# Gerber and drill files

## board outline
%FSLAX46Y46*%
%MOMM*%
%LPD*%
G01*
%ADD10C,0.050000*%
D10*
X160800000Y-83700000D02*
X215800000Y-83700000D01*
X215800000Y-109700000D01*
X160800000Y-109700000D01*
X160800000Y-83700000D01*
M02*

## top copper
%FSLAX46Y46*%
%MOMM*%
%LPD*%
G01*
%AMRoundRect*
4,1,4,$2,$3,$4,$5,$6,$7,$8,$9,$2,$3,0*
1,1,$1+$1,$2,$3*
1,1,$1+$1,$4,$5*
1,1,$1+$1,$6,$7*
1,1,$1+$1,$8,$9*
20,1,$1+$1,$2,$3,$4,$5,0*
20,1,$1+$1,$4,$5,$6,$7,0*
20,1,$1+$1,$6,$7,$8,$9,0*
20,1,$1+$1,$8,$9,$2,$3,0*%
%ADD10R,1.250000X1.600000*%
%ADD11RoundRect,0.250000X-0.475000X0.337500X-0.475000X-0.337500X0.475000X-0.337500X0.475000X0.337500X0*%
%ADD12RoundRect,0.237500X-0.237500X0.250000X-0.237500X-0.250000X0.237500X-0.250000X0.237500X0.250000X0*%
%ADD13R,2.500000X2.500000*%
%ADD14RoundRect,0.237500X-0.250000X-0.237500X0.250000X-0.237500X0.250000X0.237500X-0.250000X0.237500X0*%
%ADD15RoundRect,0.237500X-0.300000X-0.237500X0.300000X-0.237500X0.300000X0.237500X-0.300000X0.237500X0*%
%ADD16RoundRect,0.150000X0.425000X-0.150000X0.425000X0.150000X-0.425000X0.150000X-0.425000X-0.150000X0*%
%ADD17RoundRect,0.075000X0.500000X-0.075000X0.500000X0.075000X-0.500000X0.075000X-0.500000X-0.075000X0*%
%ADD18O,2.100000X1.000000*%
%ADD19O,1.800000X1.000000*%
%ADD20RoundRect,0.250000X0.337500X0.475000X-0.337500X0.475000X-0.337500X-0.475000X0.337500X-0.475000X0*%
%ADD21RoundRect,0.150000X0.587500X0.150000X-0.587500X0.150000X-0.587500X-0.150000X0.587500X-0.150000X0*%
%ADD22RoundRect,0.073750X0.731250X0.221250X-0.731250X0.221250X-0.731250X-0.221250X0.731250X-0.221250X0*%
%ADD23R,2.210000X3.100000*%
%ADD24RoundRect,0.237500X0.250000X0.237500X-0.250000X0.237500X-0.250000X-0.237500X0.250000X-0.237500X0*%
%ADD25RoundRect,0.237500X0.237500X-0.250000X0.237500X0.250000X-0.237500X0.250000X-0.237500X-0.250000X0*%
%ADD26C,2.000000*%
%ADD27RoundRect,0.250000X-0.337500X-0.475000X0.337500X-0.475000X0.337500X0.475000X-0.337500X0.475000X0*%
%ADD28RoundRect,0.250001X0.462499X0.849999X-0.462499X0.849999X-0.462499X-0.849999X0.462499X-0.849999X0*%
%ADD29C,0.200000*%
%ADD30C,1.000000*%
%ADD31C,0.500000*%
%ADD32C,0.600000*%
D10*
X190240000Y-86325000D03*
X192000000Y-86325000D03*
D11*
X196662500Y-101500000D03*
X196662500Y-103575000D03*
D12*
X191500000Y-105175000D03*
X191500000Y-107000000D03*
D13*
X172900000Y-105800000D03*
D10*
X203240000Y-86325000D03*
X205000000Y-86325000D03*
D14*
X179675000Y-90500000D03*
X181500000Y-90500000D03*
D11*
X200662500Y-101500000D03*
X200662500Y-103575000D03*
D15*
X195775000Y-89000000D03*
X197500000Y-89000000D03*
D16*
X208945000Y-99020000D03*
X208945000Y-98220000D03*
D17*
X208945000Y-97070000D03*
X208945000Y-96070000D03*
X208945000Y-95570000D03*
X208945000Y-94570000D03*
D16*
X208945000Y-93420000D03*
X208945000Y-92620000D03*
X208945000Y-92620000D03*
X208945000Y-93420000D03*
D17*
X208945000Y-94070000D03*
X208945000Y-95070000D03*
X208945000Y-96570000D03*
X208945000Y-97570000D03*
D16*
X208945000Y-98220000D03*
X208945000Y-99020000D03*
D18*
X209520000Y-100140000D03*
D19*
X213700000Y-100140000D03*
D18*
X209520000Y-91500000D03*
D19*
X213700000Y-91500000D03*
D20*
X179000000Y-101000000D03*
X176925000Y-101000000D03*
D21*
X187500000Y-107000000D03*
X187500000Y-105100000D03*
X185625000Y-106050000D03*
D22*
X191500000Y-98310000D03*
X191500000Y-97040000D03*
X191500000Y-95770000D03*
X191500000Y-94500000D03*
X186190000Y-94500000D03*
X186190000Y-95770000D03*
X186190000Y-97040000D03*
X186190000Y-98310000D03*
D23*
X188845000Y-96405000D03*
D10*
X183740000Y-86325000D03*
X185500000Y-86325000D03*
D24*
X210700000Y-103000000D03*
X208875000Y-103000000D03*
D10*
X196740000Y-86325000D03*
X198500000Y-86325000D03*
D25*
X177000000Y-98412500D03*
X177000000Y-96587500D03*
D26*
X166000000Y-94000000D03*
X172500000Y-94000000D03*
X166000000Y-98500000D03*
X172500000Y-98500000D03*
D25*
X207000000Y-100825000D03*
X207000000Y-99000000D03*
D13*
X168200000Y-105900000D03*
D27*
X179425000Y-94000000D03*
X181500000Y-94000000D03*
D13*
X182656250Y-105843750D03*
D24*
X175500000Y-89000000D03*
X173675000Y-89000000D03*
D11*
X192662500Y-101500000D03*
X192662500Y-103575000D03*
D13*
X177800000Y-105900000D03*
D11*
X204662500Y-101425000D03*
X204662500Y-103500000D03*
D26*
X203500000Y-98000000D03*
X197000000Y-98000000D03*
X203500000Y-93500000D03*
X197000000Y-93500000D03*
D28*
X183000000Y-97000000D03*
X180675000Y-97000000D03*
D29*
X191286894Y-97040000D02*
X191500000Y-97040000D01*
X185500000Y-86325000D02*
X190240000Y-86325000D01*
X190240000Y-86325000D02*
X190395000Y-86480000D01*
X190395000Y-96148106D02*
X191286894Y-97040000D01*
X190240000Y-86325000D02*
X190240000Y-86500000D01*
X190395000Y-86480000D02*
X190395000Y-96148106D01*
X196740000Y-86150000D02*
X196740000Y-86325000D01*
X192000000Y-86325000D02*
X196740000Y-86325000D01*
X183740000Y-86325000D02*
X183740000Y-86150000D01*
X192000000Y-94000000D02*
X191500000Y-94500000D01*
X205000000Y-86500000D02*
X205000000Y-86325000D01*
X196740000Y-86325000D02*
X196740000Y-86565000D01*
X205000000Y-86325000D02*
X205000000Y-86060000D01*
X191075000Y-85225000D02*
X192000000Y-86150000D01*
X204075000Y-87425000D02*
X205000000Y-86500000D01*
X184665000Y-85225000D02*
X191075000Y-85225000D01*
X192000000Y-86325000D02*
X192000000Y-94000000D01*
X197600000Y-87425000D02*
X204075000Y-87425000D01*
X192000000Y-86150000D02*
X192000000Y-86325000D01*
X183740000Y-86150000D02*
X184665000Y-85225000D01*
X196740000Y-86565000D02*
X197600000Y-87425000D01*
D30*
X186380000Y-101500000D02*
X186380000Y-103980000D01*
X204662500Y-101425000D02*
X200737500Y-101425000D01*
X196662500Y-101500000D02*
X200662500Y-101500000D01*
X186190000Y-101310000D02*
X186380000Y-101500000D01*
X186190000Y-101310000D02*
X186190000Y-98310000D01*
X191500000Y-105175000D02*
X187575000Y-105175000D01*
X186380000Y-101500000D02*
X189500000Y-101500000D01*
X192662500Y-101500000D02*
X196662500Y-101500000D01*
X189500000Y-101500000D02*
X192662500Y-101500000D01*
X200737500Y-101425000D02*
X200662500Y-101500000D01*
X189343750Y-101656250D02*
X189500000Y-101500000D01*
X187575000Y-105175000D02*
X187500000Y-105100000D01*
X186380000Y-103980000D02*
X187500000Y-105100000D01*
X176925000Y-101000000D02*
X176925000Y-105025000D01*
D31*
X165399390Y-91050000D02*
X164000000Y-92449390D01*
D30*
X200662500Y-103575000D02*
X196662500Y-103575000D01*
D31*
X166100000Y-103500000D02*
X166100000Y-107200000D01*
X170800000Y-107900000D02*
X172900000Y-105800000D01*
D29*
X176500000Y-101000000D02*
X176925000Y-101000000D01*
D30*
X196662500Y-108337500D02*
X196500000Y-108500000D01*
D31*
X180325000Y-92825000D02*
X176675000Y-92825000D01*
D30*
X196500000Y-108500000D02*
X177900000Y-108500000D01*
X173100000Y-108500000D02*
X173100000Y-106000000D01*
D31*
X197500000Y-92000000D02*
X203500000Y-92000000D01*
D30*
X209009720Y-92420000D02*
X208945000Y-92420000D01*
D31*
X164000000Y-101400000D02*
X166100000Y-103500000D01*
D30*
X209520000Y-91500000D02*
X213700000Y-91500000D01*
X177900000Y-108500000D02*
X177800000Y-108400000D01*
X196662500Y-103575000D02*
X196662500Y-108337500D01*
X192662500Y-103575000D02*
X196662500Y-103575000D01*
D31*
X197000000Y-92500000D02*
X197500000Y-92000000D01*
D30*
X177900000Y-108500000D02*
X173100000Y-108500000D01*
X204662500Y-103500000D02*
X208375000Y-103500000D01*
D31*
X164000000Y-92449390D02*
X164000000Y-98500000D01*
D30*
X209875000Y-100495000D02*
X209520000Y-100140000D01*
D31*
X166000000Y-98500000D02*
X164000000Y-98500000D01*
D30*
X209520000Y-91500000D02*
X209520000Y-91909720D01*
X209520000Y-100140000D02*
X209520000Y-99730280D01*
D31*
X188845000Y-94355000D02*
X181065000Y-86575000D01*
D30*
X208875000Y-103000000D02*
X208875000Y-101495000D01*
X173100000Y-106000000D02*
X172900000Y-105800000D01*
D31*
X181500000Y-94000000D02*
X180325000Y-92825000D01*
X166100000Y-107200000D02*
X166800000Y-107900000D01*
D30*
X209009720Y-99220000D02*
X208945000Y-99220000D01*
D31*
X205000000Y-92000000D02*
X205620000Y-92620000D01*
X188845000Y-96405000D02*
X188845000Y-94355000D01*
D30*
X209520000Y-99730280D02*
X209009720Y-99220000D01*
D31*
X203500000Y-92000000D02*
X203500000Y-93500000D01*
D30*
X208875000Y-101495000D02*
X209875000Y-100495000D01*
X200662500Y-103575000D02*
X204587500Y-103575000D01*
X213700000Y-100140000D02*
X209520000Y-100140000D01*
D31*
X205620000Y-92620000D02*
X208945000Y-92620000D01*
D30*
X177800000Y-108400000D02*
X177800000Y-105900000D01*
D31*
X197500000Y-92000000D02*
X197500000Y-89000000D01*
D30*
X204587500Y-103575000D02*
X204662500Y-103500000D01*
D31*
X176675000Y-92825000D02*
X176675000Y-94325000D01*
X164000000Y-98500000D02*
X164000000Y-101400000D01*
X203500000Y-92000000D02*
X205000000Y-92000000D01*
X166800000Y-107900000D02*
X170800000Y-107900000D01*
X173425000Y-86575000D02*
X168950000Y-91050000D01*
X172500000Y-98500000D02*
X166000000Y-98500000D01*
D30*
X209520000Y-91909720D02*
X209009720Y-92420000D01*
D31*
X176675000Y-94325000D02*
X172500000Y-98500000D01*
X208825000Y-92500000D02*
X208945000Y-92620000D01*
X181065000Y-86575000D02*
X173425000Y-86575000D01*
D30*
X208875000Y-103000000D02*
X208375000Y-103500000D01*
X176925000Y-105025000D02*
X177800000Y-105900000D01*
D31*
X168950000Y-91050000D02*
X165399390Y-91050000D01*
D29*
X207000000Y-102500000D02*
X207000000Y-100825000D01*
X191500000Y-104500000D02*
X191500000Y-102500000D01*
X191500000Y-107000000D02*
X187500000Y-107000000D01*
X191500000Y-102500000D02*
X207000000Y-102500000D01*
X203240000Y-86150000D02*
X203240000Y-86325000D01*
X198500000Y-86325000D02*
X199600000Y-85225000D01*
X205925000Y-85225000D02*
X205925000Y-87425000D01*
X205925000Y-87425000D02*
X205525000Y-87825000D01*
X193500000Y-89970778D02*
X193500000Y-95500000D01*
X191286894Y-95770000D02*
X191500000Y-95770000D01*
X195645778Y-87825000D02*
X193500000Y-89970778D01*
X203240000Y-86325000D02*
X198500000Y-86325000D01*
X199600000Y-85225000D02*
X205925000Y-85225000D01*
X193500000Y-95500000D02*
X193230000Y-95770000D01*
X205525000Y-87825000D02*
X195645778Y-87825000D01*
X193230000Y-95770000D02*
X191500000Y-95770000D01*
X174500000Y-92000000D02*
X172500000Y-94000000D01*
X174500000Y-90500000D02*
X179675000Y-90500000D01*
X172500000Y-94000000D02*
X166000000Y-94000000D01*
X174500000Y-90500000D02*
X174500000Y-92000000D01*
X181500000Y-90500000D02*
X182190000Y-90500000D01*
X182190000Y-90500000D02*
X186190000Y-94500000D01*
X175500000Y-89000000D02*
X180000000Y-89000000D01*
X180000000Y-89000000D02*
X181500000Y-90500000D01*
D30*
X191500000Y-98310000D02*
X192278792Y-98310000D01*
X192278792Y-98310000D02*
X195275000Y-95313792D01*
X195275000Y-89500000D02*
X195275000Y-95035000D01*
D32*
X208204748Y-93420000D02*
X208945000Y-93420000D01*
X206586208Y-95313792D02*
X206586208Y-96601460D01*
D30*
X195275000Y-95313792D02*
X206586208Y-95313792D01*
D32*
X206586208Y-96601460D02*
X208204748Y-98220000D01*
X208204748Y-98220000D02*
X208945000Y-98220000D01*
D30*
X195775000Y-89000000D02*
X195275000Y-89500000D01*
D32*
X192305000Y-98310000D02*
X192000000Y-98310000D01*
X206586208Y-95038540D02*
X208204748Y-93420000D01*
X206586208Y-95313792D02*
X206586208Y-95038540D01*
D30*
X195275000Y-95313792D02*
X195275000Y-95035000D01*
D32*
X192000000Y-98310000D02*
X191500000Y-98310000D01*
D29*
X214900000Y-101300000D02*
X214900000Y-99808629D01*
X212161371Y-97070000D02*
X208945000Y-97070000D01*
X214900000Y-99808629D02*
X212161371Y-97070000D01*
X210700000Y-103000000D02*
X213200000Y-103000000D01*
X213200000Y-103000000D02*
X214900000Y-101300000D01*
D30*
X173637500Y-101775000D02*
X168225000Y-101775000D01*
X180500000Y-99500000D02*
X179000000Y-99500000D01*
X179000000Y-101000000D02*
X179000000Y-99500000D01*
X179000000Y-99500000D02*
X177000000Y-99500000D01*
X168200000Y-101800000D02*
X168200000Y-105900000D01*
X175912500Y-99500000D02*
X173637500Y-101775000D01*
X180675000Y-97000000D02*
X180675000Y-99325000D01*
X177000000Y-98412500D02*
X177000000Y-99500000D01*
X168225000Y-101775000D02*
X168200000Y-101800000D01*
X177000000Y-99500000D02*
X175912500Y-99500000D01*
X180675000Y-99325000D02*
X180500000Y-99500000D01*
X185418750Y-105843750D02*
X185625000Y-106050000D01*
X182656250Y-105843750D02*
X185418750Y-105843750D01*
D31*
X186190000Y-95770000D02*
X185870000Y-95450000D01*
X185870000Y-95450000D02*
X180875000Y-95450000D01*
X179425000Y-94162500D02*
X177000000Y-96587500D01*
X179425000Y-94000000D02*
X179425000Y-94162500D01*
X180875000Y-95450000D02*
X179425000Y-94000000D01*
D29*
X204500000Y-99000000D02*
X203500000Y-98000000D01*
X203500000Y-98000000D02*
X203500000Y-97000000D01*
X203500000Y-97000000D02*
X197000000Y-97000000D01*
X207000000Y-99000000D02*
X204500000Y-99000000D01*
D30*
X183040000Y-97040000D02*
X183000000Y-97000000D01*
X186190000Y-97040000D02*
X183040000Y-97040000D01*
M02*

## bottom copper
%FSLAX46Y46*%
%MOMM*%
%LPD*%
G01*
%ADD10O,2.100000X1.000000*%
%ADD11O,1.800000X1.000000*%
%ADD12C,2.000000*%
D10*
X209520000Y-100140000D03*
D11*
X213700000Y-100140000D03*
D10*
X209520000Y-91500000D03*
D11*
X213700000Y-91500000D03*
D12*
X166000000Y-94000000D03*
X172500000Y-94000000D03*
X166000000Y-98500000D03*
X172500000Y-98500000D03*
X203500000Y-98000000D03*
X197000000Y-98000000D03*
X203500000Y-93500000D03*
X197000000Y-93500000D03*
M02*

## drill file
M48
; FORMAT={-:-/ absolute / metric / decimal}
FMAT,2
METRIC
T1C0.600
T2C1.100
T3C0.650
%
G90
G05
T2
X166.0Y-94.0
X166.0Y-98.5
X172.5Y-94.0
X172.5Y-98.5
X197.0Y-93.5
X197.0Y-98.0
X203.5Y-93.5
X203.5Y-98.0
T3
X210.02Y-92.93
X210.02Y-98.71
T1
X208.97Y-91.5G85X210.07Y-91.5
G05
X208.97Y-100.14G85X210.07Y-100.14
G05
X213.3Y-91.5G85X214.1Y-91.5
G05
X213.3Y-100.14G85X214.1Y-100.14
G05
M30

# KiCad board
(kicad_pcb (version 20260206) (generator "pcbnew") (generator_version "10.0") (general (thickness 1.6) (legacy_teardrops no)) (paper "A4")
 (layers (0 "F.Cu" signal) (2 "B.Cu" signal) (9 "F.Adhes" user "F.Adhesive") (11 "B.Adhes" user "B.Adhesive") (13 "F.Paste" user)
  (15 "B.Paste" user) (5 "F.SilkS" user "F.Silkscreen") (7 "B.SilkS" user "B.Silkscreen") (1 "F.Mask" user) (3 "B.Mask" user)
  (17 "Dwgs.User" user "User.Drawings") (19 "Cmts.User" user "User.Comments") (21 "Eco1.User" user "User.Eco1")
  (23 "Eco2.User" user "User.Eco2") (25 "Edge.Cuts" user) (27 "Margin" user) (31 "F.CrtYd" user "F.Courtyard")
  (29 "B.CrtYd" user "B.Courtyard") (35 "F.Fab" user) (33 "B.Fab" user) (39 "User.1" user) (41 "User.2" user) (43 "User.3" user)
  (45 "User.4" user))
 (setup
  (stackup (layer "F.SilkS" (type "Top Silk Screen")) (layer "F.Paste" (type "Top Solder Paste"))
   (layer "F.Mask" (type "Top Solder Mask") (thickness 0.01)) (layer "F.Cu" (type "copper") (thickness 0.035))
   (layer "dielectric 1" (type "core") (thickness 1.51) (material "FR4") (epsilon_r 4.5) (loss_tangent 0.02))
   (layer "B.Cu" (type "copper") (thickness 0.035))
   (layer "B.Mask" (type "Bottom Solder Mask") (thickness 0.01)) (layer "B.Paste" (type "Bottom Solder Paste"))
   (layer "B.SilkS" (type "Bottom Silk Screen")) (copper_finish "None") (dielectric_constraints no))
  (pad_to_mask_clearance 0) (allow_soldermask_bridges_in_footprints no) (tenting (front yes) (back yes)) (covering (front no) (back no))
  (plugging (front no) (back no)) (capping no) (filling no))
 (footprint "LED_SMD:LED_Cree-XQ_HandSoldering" (layer "F.Cu") (at 191.12 86.325)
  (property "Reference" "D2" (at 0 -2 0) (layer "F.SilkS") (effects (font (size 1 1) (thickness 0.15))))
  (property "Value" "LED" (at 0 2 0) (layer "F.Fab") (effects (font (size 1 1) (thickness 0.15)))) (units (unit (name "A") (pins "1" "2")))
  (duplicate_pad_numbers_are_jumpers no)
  (pad "1" smd rect (at -0.88 0) (size 1.25 1.6) (layers "F.Cu" "F.Mask" "F.Paste") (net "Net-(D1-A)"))
  (pad "2" smd rect (at 0.88 0) (size 1.25 1.6) (layers "F.Cu" "F.Mask" "F.Paste") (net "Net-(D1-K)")))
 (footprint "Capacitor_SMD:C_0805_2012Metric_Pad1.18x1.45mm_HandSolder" (layer "F.Cu") (at 196.6625 102.5375 -90)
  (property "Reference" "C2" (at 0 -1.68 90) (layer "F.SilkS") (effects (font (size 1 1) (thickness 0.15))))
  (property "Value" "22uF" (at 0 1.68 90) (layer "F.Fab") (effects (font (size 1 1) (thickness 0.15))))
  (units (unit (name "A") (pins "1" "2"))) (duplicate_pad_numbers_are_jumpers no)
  (pad "1" smd roundrect (at -1.0375 0 270) (size 1.175 1.45) (layers "F.Cu" "F.Mask" "F.Paste") (roundrect_rratio 0.212766) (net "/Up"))
  (pad "2" smd roundrect (at 1.0375 0 270) (size 1.175 1.45) (layers "F.Cu" "F.Mask" "F.Paste") (roundrect_rratio 0.212766) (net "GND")))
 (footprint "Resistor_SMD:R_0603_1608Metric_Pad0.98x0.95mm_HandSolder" (layer "F.Cu") (at 191.5 106.0875 -90)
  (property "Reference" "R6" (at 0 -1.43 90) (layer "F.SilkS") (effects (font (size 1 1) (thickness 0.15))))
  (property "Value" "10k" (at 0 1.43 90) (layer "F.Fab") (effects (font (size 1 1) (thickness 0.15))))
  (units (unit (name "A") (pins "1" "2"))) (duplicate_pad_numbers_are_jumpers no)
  (pad "1" smd roundrect (at -0.9125 0 270) (size 0.975 0.95) (layers "F.Cu" "F.Mask" "F.Paste") (roundrect_rratio 0.25) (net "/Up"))
  (pad "2" smd roundrect (at 0.9125 0 270) (size 0.975 0.95) (layers "F.Cu" "F.Mask" "F.Paste") (roundrect_rratio 0.25) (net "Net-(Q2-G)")))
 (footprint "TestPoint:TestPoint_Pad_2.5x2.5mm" (layer "F.Cu") (at 172.9 105.8)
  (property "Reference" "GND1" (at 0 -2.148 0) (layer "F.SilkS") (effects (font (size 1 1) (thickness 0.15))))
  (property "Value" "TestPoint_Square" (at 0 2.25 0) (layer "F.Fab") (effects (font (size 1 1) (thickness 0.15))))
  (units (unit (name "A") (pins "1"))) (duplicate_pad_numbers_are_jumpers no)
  (pad "1" smd rect (at 0 0) (size 2.5 2.5) (layers "F.Cu" "F.Mask") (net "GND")))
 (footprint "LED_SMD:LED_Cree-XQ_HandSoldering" (layer "F.Cu") (at 204.12 86.325)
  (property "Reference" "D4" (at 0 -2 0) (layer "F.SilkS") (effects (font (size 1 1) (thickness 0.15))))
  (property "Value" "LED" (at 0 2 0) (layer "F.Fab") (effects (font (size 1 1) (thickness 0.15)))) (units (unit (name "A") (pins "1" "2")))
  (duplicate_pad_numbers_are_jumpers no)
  (pad "1" smd rect (at -0.88 0) (size 1.25 1.6) (layers "F.Cu" "F.Mask" "F.Paste") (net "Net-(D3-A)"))
  (pad "2" smd rect (at 0.88 0) (size 1.25 1.6) (layers "F.Cu" "F.Mask" "F.Paste") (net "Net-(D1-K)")))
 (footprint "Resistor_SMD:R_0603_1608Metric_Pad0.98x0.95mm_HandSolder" (layer "F.Cu") (at 180.5875 90.5)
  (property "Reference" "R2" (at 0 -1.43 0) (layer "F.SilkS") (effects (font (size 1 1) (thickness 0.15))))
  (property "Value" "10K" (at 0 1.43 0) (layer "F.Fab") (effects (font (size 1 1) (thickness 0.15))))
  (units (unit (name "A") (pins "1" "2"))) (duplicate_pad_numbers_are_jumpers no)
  (pad "1" smd roundrect (at -0.9125 0) (size 0.975 0.95) (layers "F.Cu" "F.Mask" "F.Paste") (roundrect_rratio 0.25) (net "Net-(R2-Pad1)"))
  (pad "2" smd roundrect (at 0.9125 0) (size 0.975 0.95) (layers "F.Cu" "F.Mask" "F.Paste") (roundrect_rratio 0.25) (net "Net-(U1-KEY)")))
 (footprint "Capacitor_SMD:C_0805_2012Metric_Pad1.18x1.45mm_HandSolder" (layer "F.Cu") (at 200.6625 102.5375 -90)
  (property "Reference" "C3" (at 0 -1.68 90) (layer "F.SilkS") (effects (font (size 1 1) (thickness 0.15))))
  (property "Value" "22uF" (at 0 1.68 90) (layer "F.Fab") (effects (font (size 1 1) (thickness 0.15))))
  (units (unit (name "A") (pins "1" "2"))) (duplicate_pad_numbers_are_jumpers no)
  (pad "1" smd roundrect (at -1.0375 0 270) (size 1.175 1.45) (layers "F.Cu" "F.Mask" "F.Paste") (roundrect_rratio 0.212766) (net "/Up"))
  (pad "2" smd roundrect (at 1.0375 0 270) (size 1.175 1.45) (layers "F.Cu" "F.Mask" "F.Paste") (roundrect_rratio 0.212766) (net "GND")))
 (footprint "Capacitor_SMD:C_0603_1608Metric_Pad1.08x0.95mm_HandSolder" (layer "F.Cu") (at 196.6375 89)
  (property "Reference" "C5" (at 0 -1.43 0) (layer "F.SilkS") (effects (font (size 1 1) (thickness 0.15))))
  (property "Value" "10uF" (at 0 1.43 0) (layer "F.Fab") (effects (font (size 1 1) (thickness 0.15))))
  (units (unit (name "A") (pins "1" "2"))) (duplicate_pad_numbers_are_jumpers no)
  (pad "1" smd roundrect (at -0.8625 0) (size 1.075 0.95) (layers "F.Cu" "F.Mask" "F.Paste") (roundrect_rratio 0.25) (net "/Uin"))
  (pad "2" smd roundrect (at 0.8625 0) (size 1.075 0.95) (layers "F.Cu" "F.Mask" "F.Paste") (roundrect_rratio 0.25) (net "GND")))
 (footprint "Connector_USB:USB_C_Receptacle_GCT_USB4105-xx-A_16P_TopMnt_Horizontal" (layer "F.Cu") (at 212.625 95.82 90)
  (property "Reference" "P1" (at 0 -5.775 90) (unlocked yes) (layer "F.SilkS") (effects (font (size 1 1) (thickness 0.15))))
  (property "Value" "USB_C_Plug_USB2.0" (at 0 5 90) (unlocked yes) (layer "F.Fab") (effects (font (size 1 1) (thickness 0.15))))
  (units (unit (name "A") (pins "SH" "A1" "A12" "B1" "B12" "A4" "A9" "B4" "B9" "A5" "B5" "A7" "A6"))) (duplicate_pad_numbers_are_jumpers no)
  (pad "" np_thru_hole circle (at -2.89 -2.605 90) (size 0.65 0.65) (drill 0.65) (layers "*.Cu" "*.Mask"))
  (pad "" np_thru_hole circle (at 2.89 -2.605 90) (size 0.65 0.65) (drill 0.65) (layers "*.Cu" "*.Mask"))
  (pad "A1" smd roundrect (at -3.2 -3.68 90) (size 0.6 1.15) (layers "F.Cu" "F.Mask" "F.Paste") (roundrect_rratio 0.25) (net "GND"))
  (pad "A4" smd roundrect (at -2.4 -3.68 90) (size 0.6 1.15) (layers "F.Cu" "F.Mask" "F.Paste") (roundrect_rratio 0.25) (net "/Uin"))
  (pad "A5" smd roundrect (at -1.25 -3.68 90) (size 0.3 1.15) (layers "F.Cu" "F.Mask" "F.Paste") (roundrect_rratio 0.25) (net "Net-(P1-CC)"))
  (pad "A6" smd roundrect (at -0.25 -3.68 90) (size 0.3 1.15) (layers "F.Cu" "F.Mask" "F.Paste") (roundrect_rratio 0.25)
   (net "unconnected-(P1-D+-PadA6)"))
  (pad "A7" smd roundrect (at 0.25 -3.68 90) (size 0.3 1.15) (layers "F.Cu" "F.Mask" "F.Paste") (roundrect_rratio 0.25)
   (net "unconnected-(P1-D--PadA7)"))
  (pad "A8" smd roundrect (at 1.25 -3.68 90) (size 0.3 1.15) (layers "F.Cu" "F.Mask" "F.Paste") (roundrect_rratio 0.25))
  (pad "A9" smd roundrect (at 2.4 -3.68 90) (size 0.6 1.15) (layers "F.Cu" "F.Mask" "F.Paste") (roundrect_rratio 0.25) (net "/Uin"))
  (pad "A12" smd roundrect (at 3.2 -3.68 90) (size 0.6 1.15) (layers "F.Cu" "F.Mask" "F.Paste") (roundrect_rratio 0.25) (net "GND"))
  (pad "B1" smd roundrect (at 3.2 -3.68 90) (size 0.6 1.15) (layers "F.Cu" "F.Mask" "F.Paste") (roundrect_rratio 0.25) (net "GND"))
  (pad "B4" smd roundrect (at 2.4 -3.68 90) (size 0.6 1.15) (layers "F.Cu" "F.Mask" "F.Paste") (roundrect_rratio 0.25) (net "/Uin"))
  (pad "B5" smd roundrect (at 1.75 -3.68 90) (size 0.3 1.15) (layers "F.Cu" "F.Mask" "F.Paste") (roundrect_rratio 0.25)
   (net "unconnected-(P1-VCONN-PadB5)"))
  (pad "B6" smd roundrect (at 0.75 -3.68 90) (size 0.3 1.15) (layers "F.Cu" "F.Mask" "F.Paste") (roundrect_rratio 0.25))
  (pad "B7" smd roundrect (at -0.75 -3.68 90) (size 0.3 1.15) (layers "F.Cu" "F.Mask" "F.Paste") (roundrect_rratio 0.25))
  (pad "B8" smd roundrect (at -1.75 -3.68 90) (size 0.3 1.15) (layers "F.Cu" "F.Mask" "F.Paste") (roundrect_rratio 0.25))
  (pad "B9" smd roundrect (at -2.4 -3.68 90) (size 0.6 1.15) (layers "F.Cu" "F.Mask" "F.Paste") (roundrect_rratio 0.25) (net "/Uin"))
  (pad "B12" smd roundrect (at -3.2 -3.68 90) (size 0.6 1.15) (layers "F.Cu" "F.Mask" "F.Paste") (roundrect_rratio 0.25) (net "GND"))
  (pad "SH" thru_hole oval (at -4.32 -3.105 90) (size 1 2.1) (drill oval 0.6 1.7) (layers "*.Cu" "*.Mask" "F.Paste")
   (remove_unused_layers no) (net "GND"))
  (pad "SH" thru_hole oval (at -4.32 1.075 90) (size 1 1.8) (drill oval 0.6 1.4) (layers "*.Cu" "*.Mask" "F.Paste")
   (remove_unused_layers no) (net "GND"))
  (pad "SH" thru_hole oval (at 4.32 -3.105 90) (size 1 2.1) (drill oval 0.6 1.7) (layers "*.Cu" "*.Mask" "F.Paste")
   (remove_unused_layers no) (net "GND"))
  (pad "SH" thru_hole oval (at 4.32 1.075 90) (size 1 1.8) (drill oval 0.6 1.4) (layers "*.Cu" "*.Mask" "F.Paste") (remove_unused_layers no)
   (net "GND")))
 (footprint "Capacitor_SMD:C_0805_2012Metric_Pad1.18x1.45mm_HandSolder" (layer "F.Cu") (at 177.9625 101 180)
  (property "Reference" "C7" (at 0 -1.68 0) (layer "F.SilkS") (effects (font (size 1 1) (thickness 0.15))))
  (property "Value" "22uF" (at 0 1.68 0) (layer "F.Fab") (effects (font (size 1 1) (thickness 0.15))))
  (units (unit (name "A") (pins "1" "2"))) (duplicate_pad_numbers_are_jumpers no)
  (pad "1" smd roundrect (at -1.0375 0 180) (size 1.175 1.45) (layers "F.Cu" "F.Mask" "F.Paste") (roundrect_rratio 0.212766) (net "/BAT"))
  (pad "2" smd roundrect (at 1.0375 0 180) (size 1.175 1.45) (layers "F.Cu" "F.Mask" "F.Paste") (roundrect_rratio 0.212766) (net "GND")))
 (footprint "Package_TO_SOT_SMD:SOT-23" (layer "F.Cu") (at 186.5625 106.05 180)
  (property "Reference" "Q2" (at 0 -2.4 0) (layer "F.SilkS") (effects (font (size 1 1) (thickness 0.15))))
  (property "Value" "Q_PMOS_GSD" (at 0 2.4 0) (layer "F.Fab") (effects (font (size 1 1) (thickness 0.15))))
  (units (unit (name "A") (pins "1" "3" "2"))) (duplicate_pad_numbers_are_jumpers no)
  (pad "1" smd roundrect (at -0.9375 -0.95 180) (size 1.475 0.6) (layers "F.Cu" "F.Mask" "F.Paste") (roundrect_rratio 0.25)
   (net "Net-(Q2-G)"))
  (pad "2" smd roundrect (at -0.9375 0.95 180) (size 1.475 0.6) (layers "F.Cu" "F.Mask" "F.Paste") (roundrect_rratio 0.25) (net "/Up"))
  (pad "3" smd roundrect (at 0.9375 0 180) (size 1.475 0.6) (layers "F.Cu" "F.Mask" "F.Paste") (roundrect_rratio 0.25) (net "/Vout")))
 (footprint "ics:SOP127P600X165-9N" (layer "F.Cu") (at 188.845 96.405 180)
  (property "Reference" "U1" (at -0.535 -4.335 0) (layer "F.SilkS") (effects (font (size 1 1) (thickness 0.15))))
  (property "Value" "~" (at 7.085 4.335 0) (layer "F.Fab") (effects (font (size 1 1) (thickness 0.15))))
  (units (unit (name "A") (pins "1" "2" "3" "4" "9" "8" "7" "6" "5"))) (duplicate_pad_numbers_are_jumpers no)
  (pad "1" smd roundrect (at -2.655 -1.905 180) (size 1.61 0.59) (layers "F.Cu" "F.Mask" "F.Paste") (roundrect_rratio 0.125) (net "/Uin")
   (solder_mask_margin 0.102))
  (pad "2" smd roundrect (at -2.655 -0.635 180) (size 1.61 0.59) (layers "F.Cu" "F.Mask" "F.Paste") (roundrect_rratio 0.125)
   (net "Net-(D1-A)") (solder_mask_margin 0.102))
  (pad "3" smd roundrect (at -2.655 0.635 180) (size 1.61 0.59) (layers "F.Cu" "F.Mask" "F.Paste") (roundrect_rratio 0.125)
   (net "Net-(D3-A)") (solder_mask_margin 0.102))
  (pad "4" smd roundrect (at -2.655 1.905 180) (size 1.61 0.59) (layers "F.Cu" "F.Mask" "F.Paste") (roundrect_rratio 0.125)
   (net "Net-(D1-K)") (solder_mask_margin 0.102))
  (pad "5" smd roundrect (at 2.655 1.905 180) (size 1.61 0.59) (layers "F.Cu" "F.Mask" "F.Paste") (roundrect_rratio 0.125)
   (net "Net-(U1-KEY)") (solder_mask_margin 0.102))
  (pad "6" smd roundrect (at 2.655 0.635 180) (size 1.61 0.59) (layers "F.Cu" "F.Mask" "F.Paste") (roundrect_rratio 0.125) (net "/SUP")
   (solder_mask_margin 0.102))
  (pad "7" smd roundrect (at 2.655 -0.635 180) (size 1.61 0.59) (layers "F.Cu" "F.Mask" "F.Paste") (roundrect_rratio 0.125)
   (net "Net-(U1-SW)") (solder_mask_margin 0.102))
  (pad "8" smd roundrect (at 2.655 -1.905 180) (size 1.61 0.59) (layers "F.Cu" "F.Mask" "F.Paste") (roundrect_rratio 0.125) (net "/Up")
   (solder_mask_margin 0.102))
  (pad "9" smd rect (at 0 0 180) (size 2.21 3.1) (layers "F.Cu" "F.Mask") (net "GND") (solder_mask_margin 0.102)))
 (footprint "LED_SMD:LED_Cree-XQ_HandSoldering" (layer "F.Cu") (at 184.62 86.325)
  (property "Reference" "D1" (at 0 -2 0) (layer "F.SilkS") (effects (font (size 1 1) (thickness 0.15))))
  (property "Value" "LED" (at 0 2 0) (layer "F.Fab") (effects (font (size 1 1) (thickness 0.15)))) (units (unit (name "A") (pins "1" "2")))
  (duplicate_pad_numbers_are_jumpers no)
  (pad "1" smd rect (at -0.88 0) (size 1.25 1.6) (layers "F.Cu" "F.Mask" "F.Paste") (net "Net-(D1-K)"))
  (pad "2" smd rect (at 0.88 0) (size 1.25 1.6) (layers "F.Cu" "F.Mask" "F.Paste") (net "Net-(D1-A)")))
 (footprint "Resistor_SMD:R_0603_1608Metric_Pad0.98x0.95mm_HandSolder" (layer "F.Cu") (at 209.7875 103 180)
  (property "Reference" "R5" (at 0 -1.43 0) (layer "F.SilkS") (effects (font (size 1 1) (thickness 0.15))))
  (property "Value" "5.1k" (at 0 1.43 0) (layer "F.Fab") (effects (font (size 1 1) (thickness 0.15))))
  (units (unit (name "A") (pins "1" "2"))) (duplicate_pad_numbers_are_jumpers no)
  (pad "1" smd roundrect (at -0.9125 0 180) (size 0.975 0.95) (layers "F.Cu" "F.Mask" "F.Paste") (roundrect_rratio 0.25) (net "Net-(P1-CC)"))
  (pad "2" smd roundrect (at 0.9125 0 180) (size 0.975 0.95) (layers "F.Cu" "F.Mask" "F.Paste") (roundrect_rratio 0.25) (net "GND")))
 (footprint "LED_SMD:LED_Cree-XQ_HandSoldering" (layer "F.Cu") (at 197.62 86.325)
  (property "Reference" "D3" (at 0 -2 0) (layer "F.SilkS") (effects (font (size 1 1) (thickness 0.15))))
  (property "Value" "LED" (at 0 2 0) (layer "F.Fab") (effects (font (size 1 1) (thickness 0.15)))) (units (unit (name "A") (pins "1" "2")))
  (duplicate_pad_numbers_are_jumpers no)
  (pad "1" smd rect (at -0.88 0) (size 1.25 1.6) (layers "F.Cu" "F.Mask" "F.Paste") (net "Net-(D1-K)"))
  (pad "2" smd rect (at 0.88 0) (size 1.25 1.6) (layers "F.Cu" "F.Mask" "F.Paste") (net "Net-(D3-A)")))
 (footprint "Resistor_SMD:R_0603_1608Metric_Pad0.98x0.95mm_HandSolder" (layer "F.Cu") (at 177 97.5 90)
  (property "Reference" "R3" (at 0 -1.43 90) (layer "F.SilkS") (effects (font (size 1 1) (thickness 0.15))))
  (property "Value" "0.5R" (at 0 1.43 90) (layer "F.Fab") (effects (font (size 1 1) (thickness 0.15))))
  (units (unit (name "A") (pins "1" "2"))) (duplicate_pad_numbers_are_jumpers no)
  (pad "1" smd roundrect (at -0.9125 0 90) (size 0.975 0.95) (layers "F.Cu" "F.Mask" "F.Paste") (roundrect_rratio 0.25) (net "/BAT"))
  (pad "2" smd roundrect (at 0.9125 0 90) (size 0.975 0.95) (layers "F.Cu" "F.Mask" "F.Paste") (roundrect_rratio 0.25) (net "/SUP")))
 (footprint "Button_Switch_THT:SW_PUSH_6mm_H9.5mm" (layer "F.Cu") (at 166 94)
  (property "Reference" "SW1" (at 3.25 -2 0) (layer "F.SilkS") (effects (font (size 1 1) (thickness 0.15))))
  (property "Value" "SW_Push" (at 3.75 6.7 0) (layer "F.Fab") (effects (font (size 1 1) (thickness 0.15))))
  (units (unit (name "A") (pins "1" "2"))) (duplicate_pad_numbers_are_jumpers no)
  (pad "1" thru_hole circle (at 0 0 90) (size 2 2) (drill 1.1) (layers "*.Cu" "*.Mask") (remove_unused_layers no) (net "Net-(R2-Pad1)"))
  (pad "1" thru_hole circle (at 6.5 0 90) (size 2 2) (drill 1.1) (layers "*.Cu" "*.Mask") (remove_unused_layers no) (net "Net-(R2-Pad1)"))
  (pad "2" thru_hole circle (at 0 4.5 90) (size 2 2) (drill 1.1) (layers "*.Cu" "*.Mask") (remove_unused_layers no) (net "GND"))
  (pad "2" thru_hole circle (at 6.5 4.5 90) (size 2 2) (drill 1.1) (layers "*.Cu" "*.Mask") (remove_unused_layers no) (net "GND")))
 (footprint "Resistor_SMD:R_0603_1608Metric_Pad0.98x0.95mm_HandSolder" (layer "F.Cu") (at 207 99.9125 90)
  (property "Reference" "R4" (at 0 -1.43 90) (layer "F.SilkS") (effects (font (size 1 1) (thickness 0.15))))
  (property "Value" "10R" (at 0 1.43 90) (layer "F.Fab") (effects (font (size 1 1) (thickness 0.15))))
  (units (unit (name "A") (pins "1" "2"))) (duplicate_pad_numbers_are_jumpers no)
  (pad "1" smd roundrect (at -0.9125 0 90) (size 0.975 0.95) (layers "F.Cu" "F.Mask" "F.Paste") (roundrect_rratio 0.25) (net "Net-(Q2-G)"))
  (pad "2" smd roundrect (at 0.9125 0 90) (size 0.975 0.95) (layers "F.Cu" "F.Mask" "F.Paste") (roundrect_rratio 0.25) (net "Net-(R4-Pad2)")))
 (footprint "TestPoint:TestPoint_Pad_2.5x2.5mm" (layer "F.Cu") (at 168.2 105.9)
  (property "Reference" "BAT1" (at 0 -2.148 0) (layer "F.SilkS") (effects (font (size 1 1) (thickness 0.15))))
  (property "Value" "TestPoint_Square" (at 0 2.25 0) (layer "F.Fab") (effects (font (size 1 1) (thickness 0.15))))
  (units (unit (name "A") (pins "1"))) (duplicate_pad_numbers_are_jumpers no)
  (pad "1" smd rect (at 0 0) (size 2.5 2.5) (layers "F.Cu" "F.Mask") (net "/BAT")))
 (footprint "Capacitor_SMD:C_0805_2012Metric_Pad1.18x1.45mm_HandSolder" (layer "F.Cu") (at 180.4625 94)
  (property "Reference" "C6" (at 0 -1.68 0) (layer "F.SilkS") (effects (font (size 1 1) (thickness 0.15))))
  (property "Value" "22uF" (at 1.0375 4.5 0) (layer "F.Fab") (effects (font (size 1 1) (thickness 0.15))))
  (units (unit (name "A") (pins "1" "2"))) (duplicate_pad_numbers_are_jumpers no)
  (pad "1" smd roundrect (at -1.0375 0) (size 1.175 1.45) (layers "F.Cu" "F.Mask" "F.Paste") (roundrect_rratio 0.212766) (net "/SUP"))
  (pad "2" smd roundrect (at 1.0375 0) (size 1.175 1.45) (layers "F.Cu" "F.Mask" "F.Paste") (roundrect_rratio 0.212766) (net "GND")))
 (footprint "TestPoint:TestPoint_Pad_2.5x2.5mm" (layer "F.Cu") (at 182.65625 105.84375)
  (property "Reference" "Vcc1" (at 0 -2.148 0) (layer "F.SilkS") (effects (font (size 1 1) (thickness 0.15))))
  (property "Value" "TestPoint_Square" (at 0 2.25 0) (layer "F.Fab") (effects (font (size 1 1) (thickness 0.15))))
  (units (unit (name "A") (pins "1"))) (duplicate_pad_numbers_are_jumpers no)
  (pad "1" smd rect (at 0 0) (size 2.5 2.5) (layers "F.Cu" "F.Mask") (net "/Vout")))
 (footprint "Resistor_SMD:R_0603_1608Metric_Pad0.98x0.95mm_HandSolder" (layer "F.Cu") (at 174.5875 89 180)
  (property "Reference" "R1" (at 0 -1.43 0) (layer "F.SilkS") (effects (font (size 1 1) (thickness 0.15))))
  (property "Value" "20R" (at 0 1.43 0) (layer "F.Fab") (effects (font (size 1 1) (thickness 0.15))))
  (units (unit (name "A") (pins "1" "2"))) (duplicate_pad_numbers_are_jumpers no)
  (pad "1" smd roundrect (at -0.9125 0 180) (size 0.975 0.95) (layers "F.Cu" "F.Mask" "F.Paste") (roundrect_rratio 0.25)
   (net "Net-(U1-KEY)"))
  (pad "2" smd roundrect (at 0.9125 0 180) (size 0.975 0.95) (layers "F.Cu" "F.Mask" "F.Paste") (roundrect_rratio 0.25) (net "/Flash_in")))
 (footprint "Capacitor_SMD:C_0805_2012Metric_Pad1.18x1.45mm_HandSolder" (layer "F.Cu") (at 192.6625 102.5375 -90)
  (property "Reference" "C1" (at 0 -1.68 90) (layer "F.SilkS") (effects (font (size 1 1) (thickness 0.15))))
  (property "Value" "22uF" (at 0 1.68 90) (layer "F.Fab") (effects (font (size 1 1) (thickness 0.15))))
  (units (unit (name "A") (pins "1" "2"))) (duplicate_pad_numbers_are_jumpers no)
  (pad "1" smd roundrect (at -1.0375 0 270) (size 1.175 1.45) (layers "F.Cu" "F.Mask" "F.Paste") (roundrect_rratio 0.212766) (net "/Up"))
  (pad "2" smd roundrect (at 1.0375 0 270) (size 1.175 1.45) (layers "F.Cu" "F.Mask" "F.Paste") (roundrect_rratio 0.212766) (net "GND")))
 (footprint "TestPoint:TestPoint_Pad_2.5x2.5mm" (layer "F.Cu") (at 177.8 105.9)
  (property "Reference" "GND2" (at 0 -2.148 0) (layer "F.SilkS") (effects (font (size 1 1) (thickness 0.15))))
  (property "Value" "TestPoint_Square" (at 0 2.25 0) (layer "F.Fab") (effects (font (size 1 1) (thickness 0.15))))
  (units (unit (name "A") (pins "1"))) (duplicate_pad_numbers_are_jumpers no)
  (pad "1" smd rect (at 0 0) (size 2.5 2.5) (layers "F.Cu" "F.Mask") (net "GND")))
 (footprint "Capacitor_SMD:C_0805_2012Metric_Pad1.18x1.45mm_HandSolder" (layer "F.Cu") (at 204.6625 102.4625 -90)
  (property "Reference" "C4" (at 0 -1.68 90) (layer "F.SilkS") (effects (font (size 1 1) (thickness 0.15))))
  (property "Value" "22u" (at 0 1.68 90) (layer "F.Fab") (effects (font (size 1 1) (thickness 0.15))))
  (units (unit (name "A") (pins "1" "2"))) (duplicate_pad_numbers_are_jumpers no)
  (pad "1" smd roundrect (at -1.0375 0 270) (size 1.175 1.45) (layers "F.Cu" "F.Mask" "F.Paste") (roundrect_rratio 0.212766) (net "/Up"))
  (pad "2" smd roundrect (at 1.0375 0 270) (size 1.175 1.45) (layers "F.Cu" "F.Mask" "F.Paste") (roundrect_rratio 0.212766) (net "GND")))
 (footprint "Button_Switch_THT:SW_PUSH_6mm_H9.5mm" (layer "F.Cu") (at 203.5 98 180)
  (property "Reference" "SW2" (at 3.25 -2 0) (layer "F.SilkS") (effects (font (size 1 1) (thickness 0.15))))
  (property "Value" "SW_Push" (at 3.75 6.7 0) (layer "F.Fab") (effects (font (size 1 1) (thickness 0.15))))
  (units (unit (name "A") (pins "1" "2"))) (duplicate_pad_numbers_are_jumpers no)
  (pad "1" thru_hole circle (at 0 0 270) (size 2 2) (drill 1.1) (layers "*.Cu" "*.Mask") (remove_unused_layers no) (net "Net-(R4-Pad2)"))
  (pad "1" thru_hole circle (at 6.5 0 270) (size 2 2) (drill 1.1) (layers "*.Cu" "*.Mask") (remove_unused_layers no) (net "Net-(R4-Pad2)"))
  (pad "2" thru_hole circle (at 0 4.5 270) (size 2 2) (drill 1.1) (layers "*.Cu" "*.Mask") (remove_unused_layers no) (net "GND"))
  (pad "2" thru_hole circle (at 6.5 4.5 270) (size 2 2) (drill 1.1) (layers "*.Cu" "*.Mask") (remove_unused_layers no) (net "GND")))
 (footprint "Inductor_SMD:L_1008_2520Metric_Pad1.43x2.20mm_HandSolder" (layer "F.Cu") (at 181.8375 97 180)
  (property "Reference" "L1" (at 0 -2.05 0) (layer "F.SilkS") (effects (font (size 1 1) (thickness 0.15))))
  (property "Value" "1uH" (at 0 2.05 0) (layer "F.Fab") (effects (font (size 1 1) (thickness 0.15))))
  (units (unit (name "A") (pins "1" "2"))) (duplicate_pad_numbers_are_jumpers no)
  (pad "1" smd roundrect (at -1.1625 0 180) (size 1.425 2.2) (layers "F.Cu" "F.Mask" "F.Paste") (roundrect_rratio 0.175439)
   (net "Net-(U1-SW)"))
  (pad "2" smd roundrect (at 1.1625 0 180) (size 1.425 2.2) (layers "F.Cu" "F.Mask" "F.Paste") (roundrect_rratio 0.175439) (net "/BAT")))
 (gr_rect (start 160.8 83.7) (end 215.8 109.7) (stroke (width 0.05) (type solid)) (fill no) (layer "Edge.Cuts"))
 (segment (start 191.286894 97.04) (end 191.5 97.04) (width 0.2) (layer "F.Cu") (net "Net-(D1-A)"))
 (segment (start 185.5 86.325) (end 190.24 86.325) (width 0.2) (layer "F.Cu") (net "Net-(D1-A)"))
 (segment (start 190.24 86.325) (end 190.395 86.48) (width 0.2) (layer "F.Cu") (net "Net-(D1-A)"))
 (segment (start 190.395 96.148106) (end 191.286894 97.04) (width 0.2) (layer "F.Cu") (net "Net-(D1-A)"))
 (segment (start 190.24 86.325) (end 190.24 86.5) (width 0.2) (layer "F.Cu") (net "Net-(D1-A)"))
 (segment (start 190.395 86.48) (end 190.395 96.148106) (width 0.2) (layer "F.Cu") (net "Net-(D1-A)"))
 (segment (start 196.74 86.15) (end 196.74 86.325) (width 0.2) (layer "F.Cu") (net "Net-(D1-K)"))
 (segment (start 192 86.325) (end 196.74 86.325) (width 0.2) (layer "F.Cu") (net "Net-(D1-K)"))
 (segment (start 183.74 86.325) (end 183.74 86.15) (width 0.2) (layer "F.Cu") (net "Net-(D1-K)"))
 (segment (start 192 94) (end 191.5 94.5) (width 0.2) (layer "F.Cu") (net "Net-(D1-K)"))
 (segment (start 205 86.5) (end 205 86.325) (width 0.2) (layer "F.Cu") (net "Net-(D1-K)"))
 (segment (start 196.74 86.325) (end 196.74 86.565) (width 0.2) (layer "F.Cu") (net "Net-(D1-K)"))
 (segment (start 205 86.325) (end 205 86.06) (width 0.2) (layer "F.Cu") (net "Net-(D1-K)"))
 (segment (start 191.075 85.225) (end 192 86.15) (width 0.2) (layer "F.Cu") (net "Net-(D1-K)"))
 (segment (start 204.075 87.425) (end 205 86.5) (width 0.2) (layer "F.Cu") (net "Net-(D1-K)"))
 (segment (start 184.665 85.225) (end 191.075 85.225) (width 0.2) (layer "F.Cu") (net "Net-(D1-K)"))
 (segment (start 192 86.325) (end 192 94) (width 0.2) (layer "F.Cu") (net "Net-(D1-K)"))
 (segment (start 197.6 87.425) (end 204.075 87.425) (width 0.2) (layer "F.Cu") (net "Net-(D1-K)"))
 (segment (start 192 86.15) (end 192 86.325) (width 0.2) (layer "F.Cu") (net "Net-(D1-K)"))
 (segment (start 183.74 86.15) (end 184.665 85.225) (width 0.2) (layer "F.Cu") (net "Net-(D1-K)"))
 (segment (start 196.74 86.565) (end 197.6 87.425) (width 0.2) (layer "F.Cu") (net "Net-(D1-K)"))
 (segment (start 186.38 101.5) (end 186.38 103.98) (width 1) (layer "F.Cu") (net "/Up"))
 (segment (start 204.6625 101.425) (end 200.7375 101.425) (width 1) (layer "F.Cu") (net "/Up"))
 (segment (start 196.6625 101.5) (end 200.6625 101.5) (width 1) (layer "F.Cu") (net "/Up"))
 (segment (start 186.19 101.31) (end 186.38 101.5) (width 1) (layer "F.Cu") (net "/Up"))
 (segment (start 186.19 101.31) (end 186.19 98.31) (width 1) (layer "F.Cu") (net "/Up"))
 (segment (start 191.5 105.175) (end 187.575 105.175) (width 1) (layer "F.Cu") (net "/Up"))
 (segment (start 186.38 101.5) (end 189.5 101.5) (width 1) (layer "F.Cu") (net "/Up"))
 (segment (start 192.6625 101.5) (end 196.6625 101.5) (width 1) (layer "F.Cu") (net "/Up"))
 (segment (start 189.5 101.5) (end 192.6625 101.5) (width 1) (layer "F.Cu") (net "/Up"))
 (segment (start 200.7375 101.425) (end 200.6625 101.5) (width 1) (layer "F.Cu") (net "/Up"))
 (segment (start 189.34375 101.65625) (end 189.5 101.5) (width 1) (layer "F.Cu") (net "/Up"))
 (segment (start 187.575 105.175) (end 187.5 105.1) (width 1) (layer "F.Cu") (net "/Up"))
 (segment (start 186.38 103.98) (end 187.5 105.1) (width 1) (layer "F.Cu") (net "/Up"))
 (segment (start 176.925 101) (end 176.925 105.025) (width 1) (layer "F.Cu") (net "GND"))
 (segment (start 165.39939 91.05) (end 164 92.44939) (width 0.5) (layer "F.Cu") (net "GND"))
 (segment (start 200.6625 103.575) (end 196.6625 103.575) (width 1) (layer "F.Cu") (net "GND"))
 (segment (start 166.1 103.5) (end 166.1 107.2) (width 0.5) (layer "F.Cu") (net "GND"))
 (segment (start 170.8 107.9) (end 172.9 105.8) (width 0.5) (layer "F.Cu") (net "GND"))
 (segment (start 176.5 101) (end 176.925 101) (width 0.2) (layer "F.Cu") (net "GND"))
 (segment (start 196.6625 108.3375) (end 196.5 108.5) (width 1) (layer "F.Cu") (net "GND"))
 (segment (start 180.325 92.825) (end 176.675 92.825) (width 0.5) (layer "F.Cu") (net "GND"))
 (segment (start 196.5 108.5) (end 177.9 108.5) (width 1) (layer "F.Cu") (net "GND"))
 (segment (start 173.1 108.5) (end 173.1 106) (width 1) (layer "F.Cu") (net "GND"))
 (segment (start 197.5 92) (end 203.5 92) (width 0.5) (layer "F.Cu") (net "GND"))
 (segment (start 209.00972 92.42) (end 208.945 92.42) (width 1) (layer "F.Cu") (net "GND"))
 (segment (start 164 101.4) (end 166.1 103.5) (width 0.5) (layer "F.Cu") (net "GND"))
 (segment (start 209.52 91.5) (end 213.7 91.5) (width 1) (layer "F.Cu") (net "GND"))
 (segment (start 177.9 108.5) (end 177.8 108.4) (width 1) (layer "F.Cu") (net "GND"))
 (segment (start 196.6625 103.575) (end 196.6625 108.3375) (width 1) (layer "F.Cu") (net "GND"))
 (segment (start 192.6625 103.575) (end 196.6625 103.575) (width 1) (layer "F.Cu") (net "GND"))
 (segment (start 197 92.5) (end 197.5 92) (width 0.5) (layer "F.Cu") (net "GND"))
 (segment (start 177.9 108.5) (end 173.1 108.5) (width 1) (layer "F.Cu") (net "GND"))
 (segment (start 204.6625 103.5) (end 208.375 103.5) (width 1) (layer "F.Cu") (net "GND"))
 (segment (start 164 92.44939) (end 164 98.5) (width 0.5) (layer "F.Cu") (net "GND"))
 (segment (start 209.875 100.495) (end 209.52 100.14) (width 1) (layer "F.Cu") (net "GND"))
 (segment (start 166 98.5) (end 164 98.5) (width 0.5) (layer "F.Cu") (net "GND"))
 (segment (start 209.52 91.5) (end 209.52 91.90972) (width 1) (layer "F.Cu") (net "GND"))
 (segment (start 209.52 100.14) (end 209.52 99.73028) (width 1) (layer "F.Cu") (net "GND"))
 (segment (start 188.845 94.355) (end 181.065 86.575) (width 0.5) (layer "F.Cu") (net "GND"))
 (segment (start 208.875 103) (end 208.875 101.495) (width 1) (layer "F.Cu") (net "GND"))
 (segment (start 173.1 106) (end 172.9 105.8) (width 1) (layer "F.Cu") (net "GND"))
 (segment (start 181.5 94) (end 180.325 92.825) (width 0.5) (layer "F.Cu") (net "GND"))
 (segment (start 166.1 107.2) (end 166.8 107.9) (width 0.5) (layer "F.Cu") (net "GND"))
 (segment (start 209.00972 99.22) (end 208.945 99.22) (width 1) (layer "F.Cu") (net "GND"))
 (segment (start 205 92) (end 205.62 92.62) (width 0.5) (layer "F.Cu") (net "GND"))
 (segment (start 188.845 96.405) (end 188.845 94.355) (width 0.5) (layer "F.Cu") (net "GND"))
 (segment (start 209.52 99.73028) (end 209.00972 99.22) (width 1) (layer "F.Cu") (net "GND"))
 (segment (start 203.5 92) (end 203.5 93.5) (width 0.5) (layer "F.Cu") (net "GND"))
 (segment (start 208.875 101.495) (end 209.875 100.495) (width 1) (layer "F.Cu") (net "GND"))
 (segment (start 200.6625 103.575) (end 204.5875 103.575) (width 1) (layer "F.Cu") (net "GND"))
 (segment (start 213.7 100.14) (end 209.52 100.14) (width 1) (layer "F.Cu") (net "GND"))
 (segment (start 205.62 92.62) (end 208.945 92.62) (width 0.5) (layer "F.Cu") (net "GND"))
 (segment (start 177.8 108.4) (end 177.8 105.9) (width 1) (layer "F.Cu") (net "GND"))
 (segment (start 197.5 92) (end 197.5 89) (width 0.5) (layer "F.Cu") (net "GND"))
 (segment (start 204.5875 103.575) (end 204.6625 103.5) (width 1) (layer "F.Cu") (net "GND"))
 (segment (start 176.675 92.825) (end 176.675 94.325) (width 0.5) (layer "F.Cu") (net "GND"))
 (segment (start 164 98.5) (end 164 101.4) (width 0.5) (layer "F.Cu") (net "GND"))
 (segment (start 203.5 92) (end 205 92) (width 0.5) (layer "F.Cu") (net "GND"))
 (segment (start 166.8 107.9) (end 170.8 107.9) (width 0.5) (layer "F.Cu") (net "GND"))
 (segment (start 173.425 86.575) (end 168.95 91.05) (width 0.5) (layer "F.Cu") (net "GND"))
 (segment (start 172.5 98.5) (end 166 98.5) (width 0.5) (layer "F.Cu") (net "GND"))
 (segment (start 209.52 91.90972) (end 209.00972 92.42) (width 1) (layer "F.Cu") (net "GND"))
 (segment (start 176.675 94.325) (end 172.5 98.5) (width 0.5) (layer "F.Cu") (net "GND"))
 (segment (start 208.825 92.5) (end 208.945 92.62) (width 0.5) (layer "F.Cu") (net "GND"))
 (segment (start 181.065 86.575) (end 173.425 86.575) (width 0.5) (layer "F.Cu") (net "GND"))
 (segment (start 208.875 103) (end 208.375 103.5) (width 1) (layer "F.Cu") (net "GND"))
 (segment (start 176.925 105.025) (end 177.8 105.9) (width 1) (layer "F.Cu") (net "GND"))
 (segment (start 168.95 91.05) (end 165.39939 91.05) (width 0.5) (layer "F.Cu") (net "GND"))
 (segment (start 207 102.5) (end 207 100.825) (width 0.2) (layer "F.Cu") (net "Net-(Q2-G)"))
 (segment (start 191.5 104.5) (end 191.5 102.5) (width 0.2) (layer "F.Cu") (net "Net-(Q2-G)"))
 (segment (start 191.5 107) (end 187.5 107) (width 0.2) (layer "F.Cu") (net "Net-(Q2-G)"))
 (segment (start 191.5 102.5) (end 207 102.5) (width 0.2) (layer "F.Cu") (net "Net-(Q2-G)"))
 (segment (start 203.24 86.15) (end 203.24 86.325) (width 0.2) (layer "F.Cu") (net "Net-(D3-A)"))
 (segment (start 198.5 86.325) (end 199.6 85.225) (width 0.2) (layer "F.Cu") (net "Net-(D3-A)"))
 (segment (start 205.925 85.225) (end 205.925 87.425) (width 0.2) (layer "F.Cu") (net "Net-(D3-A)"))
 (segment (start 205.925 87.425) (end 205.525 87.825) (width 0.2) (layer "F.Cu") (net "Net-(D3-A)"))
 (segment (start 193.5 89.970778) (end 193.5 95.5) (width 0.2) (layer "F.Cu") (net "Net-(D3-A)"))
 (segment (start 191.286894 95.77) (end 191.5 95.77) (width 0.2) (layer "F.Cu") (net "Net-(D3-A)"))
 (segment (start 195.645778 87.825) (end 193.5 89.970778) (width 0.2) (layer "F.Cu") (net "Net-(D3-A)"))
 (segment (start 203.24 86.325) (end 198.5 86.325) (width 0.2) (layer "F.Cu") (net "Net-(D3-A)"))
 (segment (start 199.6 85.225) (end 205.925 85.225) (width 0.2) (layer "F.Cu") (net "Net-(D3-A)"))
 (segment (start 193.5 95.5) (end 193.23 95.77) (width 0.2) (layer "F.Cu") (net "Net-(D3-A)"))
 (segment (start 205.525 87.825) (end 195.645778 87.825) (width 0.2) (layer "F.Cu") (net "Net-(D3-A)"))
 (segment (start 193.23 95.77) (end 191.5 95.77) (width 0.2) (layer "F.Cu") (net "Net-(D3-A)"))
 (segment (start 174.5 92) (end 172.5 94) (width 0.2) (layer "F.Cu") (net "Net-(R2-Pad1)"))
 (segment (start 174.5 90.5) (end 179.675 90.5) (width 0.2) (layer "F.Cu") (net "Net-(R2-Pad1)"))
 (segment (start 172.5 94) (end 166 94) (width 0.2) (layer "F.Cu") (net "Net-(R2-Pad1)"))
 (segment (start 174.5 90.5) (end 174.5 92) (width 0.2) (layer "F.Cu") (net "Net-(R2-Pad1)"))
 (segment (start 181.5 90.5) (end 182.19 90.5) (width 0.2) (layer "F.Cu") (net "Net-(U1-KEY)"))
 (segment (start 182.19 90.5) (end 186.19 94.5) (width 0.2) (layer "F.Cu") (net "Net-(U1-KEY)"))
 (segment (start 175.5 89) (end 180 89) (width 0.2) (layer "F.Cu") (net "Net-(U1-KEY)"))
 (segment (start 180 89) (end 181.5 90.5) (width 0.2) (layer "F.Cu") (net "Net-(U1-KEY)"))
 (segment (start 191.5 98.31) (end 192.278792 98.31) (width 1) (layer "F.Cu") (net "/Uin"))
 (segment (start 192.278792 98.31) (end 195.275 95.313792) (width 1) (layer "F.Cu") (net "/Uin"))
 (segment (start 195.275 89.5) (end 195.275 95.035) (width 1) (layer "F.Cu") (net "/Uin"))
 (segment (start 208.204748 93.42) (end 208.945 93.42) (width 0.6) (layer "F.Cu") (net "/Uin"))
 (segment (start 206.586208 95.313792) (end 206.586208 96.60146) (width 0.6) (layer "F.Cu") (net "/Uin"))
 (segment (start 195.275 95.313792) (end 206.586208 95.313792) (width 1) (layer "F.Cu") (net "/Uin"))
 (segment (start 206.586208 96.60146) (end 208.204748 98.22) (width 0.6) (layer "F.Cu") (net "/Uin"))
 (segment (start 208.204748 98.22) (end 208.945 98.22) (width 0.6) (layer "F.Cu") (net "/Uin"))
 (segment (start 195.775 89) (end 195.275 89.5) (width 1) (layer "F.Cu") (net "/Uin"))
 (segment (start 192.305 98.31) (end 192 98.31) (width 0.6) (layer "F.Cu") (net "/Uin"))
 (segment (start 206.586208 95.03854) (end 208.204748 93.42) (width 0.6) (layer "F.Cu") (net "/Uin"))
 (segment (start 206.586208 95.313792) (end 206.586208 95.03854) (width 0.6) (layer "F.Cu") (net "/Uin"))
 (segment (start 195.275 95.313792) (end 195.275 95.035) (width 1) (layer "F.Cu") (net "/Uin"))
 (segment (start 192 98.31) (end 191.5 98.31) (width 0.6) (layer "F.Cu") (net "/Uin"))
 (segment (start 214.9 101.3) (end 214.9 99.808629) (width 0.2) (layer "F.Cu") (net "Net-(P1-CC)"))
 (segment (start 212.161371 97.07) (end 208.945 97.07) (width 0.2) (layer "F.Cu") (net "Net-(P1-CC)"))
 (segment (start 214.9 99.808629) (end 212.161371 97.07) (width 0.2) (layer "F.Cu") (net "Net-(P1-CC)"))
 (segment (start 210.7 103) (end 213.2 103) (width 0.2) (layer "F.Cu") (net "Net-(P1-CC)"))
 (segment (start 213.2 103) (end 214.9 101.3) (width 0.2) (layer "F.Cu") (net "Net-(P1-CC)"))
 (segment (start 173.6375 101.775) (end 168.225 101.775) (width 1) (layer "F.Cu") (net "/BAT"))
 (segment (start 180.5 99.5) (end 179 99.5) (width 1) (layer "F.Cu") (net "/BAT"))
 (segment (start 179 101) (end 179 99.5) (width 1) (layer "F.Cu") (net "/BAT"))
 (segment (start 179 99.5) (end 177 99.5) (width 1) (layer "F.Cu") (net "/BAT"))
 (segment (start 168.2 101.8) (end 168.2 105.9) (width 1) (layer "F.Cu") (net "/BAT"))
 (segment (start 175.9125 99.5) (end 173.6375 101.775) (width 1) (layer "F.Cu") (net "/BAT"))
 (segment (start 180.675 97) (end 180.675 99.325) (width 1) (layer "F.Cu") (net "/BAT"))
 (segment (start 177 98.4125) (end 177 99.5) (width 1) (layer "F.Cu") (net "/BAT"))
 (segment (start 168.225 101.775) (end 168.2 101.8) (width 1) (layer "F.Cu") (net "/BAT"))
 (segment (start 177 99.5) (end 175.9125 99.5) (width 1) (layer "F.Cu") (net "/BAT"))
 (segment (start 180.675 99.325) (end 180.5 99.5) (width 1) (layer "F.Cu") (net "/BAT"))
 (segment (start 185.41875 105.84375) (end 185.625 106.05) (width 1) (layer "F.Cu") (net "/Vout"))
 (segment (start 182.65625 105.84375) (end 185.41875 105.84375) (width 1) (layer "F.Cu") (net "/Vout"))
 (segment (start 186.19 95.77) (end 185.87 95.45) (width 0.5) (layer "F.Cu") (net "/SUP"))
 (segment (start 185.87 95.45) (end 180.875 95.45) (width 0.5) (layer "F.Cu") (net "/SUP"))
 (segment (start 179.425 94.1625) (end 177 96.5875) (width 0.5) (layer "F.Cu") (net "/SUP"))
 (segment (start 179.425 94) (end 179.425 94.1625) (width 0.5) (layer "F.Cu") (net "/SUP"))
 (segment (start 180.875 95.45) (end 179.425 94) (width 0.5) (layer "F.Cu") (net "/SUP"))
 (segment (start 204.5 99) (end 203.5 98) (width 0.2) (layer "F.Cu") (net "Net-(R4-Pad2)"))
 (segment (start 203.5 98) (end 203.5 97) (width 0.2) (layer "F.Cu") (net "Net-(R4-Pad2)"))
 (segment (start 203.5 97) (end 197 97) (width 0.2) (layer "F.Cu") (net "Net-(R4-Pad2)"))
 (segment (start 207 99) (end 204.5 99) (width 0.2) (layer "F.Cu") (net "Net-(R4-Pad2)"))
 (segment (start 183.04 97.04) (end 183 97) (width 1) (layer "F.Cu") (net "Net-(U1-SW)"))
 (segment (start 186.19 97.04) (end 183.04 97.04) (width 1) (layer "F.Cu") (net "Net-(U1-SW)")))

